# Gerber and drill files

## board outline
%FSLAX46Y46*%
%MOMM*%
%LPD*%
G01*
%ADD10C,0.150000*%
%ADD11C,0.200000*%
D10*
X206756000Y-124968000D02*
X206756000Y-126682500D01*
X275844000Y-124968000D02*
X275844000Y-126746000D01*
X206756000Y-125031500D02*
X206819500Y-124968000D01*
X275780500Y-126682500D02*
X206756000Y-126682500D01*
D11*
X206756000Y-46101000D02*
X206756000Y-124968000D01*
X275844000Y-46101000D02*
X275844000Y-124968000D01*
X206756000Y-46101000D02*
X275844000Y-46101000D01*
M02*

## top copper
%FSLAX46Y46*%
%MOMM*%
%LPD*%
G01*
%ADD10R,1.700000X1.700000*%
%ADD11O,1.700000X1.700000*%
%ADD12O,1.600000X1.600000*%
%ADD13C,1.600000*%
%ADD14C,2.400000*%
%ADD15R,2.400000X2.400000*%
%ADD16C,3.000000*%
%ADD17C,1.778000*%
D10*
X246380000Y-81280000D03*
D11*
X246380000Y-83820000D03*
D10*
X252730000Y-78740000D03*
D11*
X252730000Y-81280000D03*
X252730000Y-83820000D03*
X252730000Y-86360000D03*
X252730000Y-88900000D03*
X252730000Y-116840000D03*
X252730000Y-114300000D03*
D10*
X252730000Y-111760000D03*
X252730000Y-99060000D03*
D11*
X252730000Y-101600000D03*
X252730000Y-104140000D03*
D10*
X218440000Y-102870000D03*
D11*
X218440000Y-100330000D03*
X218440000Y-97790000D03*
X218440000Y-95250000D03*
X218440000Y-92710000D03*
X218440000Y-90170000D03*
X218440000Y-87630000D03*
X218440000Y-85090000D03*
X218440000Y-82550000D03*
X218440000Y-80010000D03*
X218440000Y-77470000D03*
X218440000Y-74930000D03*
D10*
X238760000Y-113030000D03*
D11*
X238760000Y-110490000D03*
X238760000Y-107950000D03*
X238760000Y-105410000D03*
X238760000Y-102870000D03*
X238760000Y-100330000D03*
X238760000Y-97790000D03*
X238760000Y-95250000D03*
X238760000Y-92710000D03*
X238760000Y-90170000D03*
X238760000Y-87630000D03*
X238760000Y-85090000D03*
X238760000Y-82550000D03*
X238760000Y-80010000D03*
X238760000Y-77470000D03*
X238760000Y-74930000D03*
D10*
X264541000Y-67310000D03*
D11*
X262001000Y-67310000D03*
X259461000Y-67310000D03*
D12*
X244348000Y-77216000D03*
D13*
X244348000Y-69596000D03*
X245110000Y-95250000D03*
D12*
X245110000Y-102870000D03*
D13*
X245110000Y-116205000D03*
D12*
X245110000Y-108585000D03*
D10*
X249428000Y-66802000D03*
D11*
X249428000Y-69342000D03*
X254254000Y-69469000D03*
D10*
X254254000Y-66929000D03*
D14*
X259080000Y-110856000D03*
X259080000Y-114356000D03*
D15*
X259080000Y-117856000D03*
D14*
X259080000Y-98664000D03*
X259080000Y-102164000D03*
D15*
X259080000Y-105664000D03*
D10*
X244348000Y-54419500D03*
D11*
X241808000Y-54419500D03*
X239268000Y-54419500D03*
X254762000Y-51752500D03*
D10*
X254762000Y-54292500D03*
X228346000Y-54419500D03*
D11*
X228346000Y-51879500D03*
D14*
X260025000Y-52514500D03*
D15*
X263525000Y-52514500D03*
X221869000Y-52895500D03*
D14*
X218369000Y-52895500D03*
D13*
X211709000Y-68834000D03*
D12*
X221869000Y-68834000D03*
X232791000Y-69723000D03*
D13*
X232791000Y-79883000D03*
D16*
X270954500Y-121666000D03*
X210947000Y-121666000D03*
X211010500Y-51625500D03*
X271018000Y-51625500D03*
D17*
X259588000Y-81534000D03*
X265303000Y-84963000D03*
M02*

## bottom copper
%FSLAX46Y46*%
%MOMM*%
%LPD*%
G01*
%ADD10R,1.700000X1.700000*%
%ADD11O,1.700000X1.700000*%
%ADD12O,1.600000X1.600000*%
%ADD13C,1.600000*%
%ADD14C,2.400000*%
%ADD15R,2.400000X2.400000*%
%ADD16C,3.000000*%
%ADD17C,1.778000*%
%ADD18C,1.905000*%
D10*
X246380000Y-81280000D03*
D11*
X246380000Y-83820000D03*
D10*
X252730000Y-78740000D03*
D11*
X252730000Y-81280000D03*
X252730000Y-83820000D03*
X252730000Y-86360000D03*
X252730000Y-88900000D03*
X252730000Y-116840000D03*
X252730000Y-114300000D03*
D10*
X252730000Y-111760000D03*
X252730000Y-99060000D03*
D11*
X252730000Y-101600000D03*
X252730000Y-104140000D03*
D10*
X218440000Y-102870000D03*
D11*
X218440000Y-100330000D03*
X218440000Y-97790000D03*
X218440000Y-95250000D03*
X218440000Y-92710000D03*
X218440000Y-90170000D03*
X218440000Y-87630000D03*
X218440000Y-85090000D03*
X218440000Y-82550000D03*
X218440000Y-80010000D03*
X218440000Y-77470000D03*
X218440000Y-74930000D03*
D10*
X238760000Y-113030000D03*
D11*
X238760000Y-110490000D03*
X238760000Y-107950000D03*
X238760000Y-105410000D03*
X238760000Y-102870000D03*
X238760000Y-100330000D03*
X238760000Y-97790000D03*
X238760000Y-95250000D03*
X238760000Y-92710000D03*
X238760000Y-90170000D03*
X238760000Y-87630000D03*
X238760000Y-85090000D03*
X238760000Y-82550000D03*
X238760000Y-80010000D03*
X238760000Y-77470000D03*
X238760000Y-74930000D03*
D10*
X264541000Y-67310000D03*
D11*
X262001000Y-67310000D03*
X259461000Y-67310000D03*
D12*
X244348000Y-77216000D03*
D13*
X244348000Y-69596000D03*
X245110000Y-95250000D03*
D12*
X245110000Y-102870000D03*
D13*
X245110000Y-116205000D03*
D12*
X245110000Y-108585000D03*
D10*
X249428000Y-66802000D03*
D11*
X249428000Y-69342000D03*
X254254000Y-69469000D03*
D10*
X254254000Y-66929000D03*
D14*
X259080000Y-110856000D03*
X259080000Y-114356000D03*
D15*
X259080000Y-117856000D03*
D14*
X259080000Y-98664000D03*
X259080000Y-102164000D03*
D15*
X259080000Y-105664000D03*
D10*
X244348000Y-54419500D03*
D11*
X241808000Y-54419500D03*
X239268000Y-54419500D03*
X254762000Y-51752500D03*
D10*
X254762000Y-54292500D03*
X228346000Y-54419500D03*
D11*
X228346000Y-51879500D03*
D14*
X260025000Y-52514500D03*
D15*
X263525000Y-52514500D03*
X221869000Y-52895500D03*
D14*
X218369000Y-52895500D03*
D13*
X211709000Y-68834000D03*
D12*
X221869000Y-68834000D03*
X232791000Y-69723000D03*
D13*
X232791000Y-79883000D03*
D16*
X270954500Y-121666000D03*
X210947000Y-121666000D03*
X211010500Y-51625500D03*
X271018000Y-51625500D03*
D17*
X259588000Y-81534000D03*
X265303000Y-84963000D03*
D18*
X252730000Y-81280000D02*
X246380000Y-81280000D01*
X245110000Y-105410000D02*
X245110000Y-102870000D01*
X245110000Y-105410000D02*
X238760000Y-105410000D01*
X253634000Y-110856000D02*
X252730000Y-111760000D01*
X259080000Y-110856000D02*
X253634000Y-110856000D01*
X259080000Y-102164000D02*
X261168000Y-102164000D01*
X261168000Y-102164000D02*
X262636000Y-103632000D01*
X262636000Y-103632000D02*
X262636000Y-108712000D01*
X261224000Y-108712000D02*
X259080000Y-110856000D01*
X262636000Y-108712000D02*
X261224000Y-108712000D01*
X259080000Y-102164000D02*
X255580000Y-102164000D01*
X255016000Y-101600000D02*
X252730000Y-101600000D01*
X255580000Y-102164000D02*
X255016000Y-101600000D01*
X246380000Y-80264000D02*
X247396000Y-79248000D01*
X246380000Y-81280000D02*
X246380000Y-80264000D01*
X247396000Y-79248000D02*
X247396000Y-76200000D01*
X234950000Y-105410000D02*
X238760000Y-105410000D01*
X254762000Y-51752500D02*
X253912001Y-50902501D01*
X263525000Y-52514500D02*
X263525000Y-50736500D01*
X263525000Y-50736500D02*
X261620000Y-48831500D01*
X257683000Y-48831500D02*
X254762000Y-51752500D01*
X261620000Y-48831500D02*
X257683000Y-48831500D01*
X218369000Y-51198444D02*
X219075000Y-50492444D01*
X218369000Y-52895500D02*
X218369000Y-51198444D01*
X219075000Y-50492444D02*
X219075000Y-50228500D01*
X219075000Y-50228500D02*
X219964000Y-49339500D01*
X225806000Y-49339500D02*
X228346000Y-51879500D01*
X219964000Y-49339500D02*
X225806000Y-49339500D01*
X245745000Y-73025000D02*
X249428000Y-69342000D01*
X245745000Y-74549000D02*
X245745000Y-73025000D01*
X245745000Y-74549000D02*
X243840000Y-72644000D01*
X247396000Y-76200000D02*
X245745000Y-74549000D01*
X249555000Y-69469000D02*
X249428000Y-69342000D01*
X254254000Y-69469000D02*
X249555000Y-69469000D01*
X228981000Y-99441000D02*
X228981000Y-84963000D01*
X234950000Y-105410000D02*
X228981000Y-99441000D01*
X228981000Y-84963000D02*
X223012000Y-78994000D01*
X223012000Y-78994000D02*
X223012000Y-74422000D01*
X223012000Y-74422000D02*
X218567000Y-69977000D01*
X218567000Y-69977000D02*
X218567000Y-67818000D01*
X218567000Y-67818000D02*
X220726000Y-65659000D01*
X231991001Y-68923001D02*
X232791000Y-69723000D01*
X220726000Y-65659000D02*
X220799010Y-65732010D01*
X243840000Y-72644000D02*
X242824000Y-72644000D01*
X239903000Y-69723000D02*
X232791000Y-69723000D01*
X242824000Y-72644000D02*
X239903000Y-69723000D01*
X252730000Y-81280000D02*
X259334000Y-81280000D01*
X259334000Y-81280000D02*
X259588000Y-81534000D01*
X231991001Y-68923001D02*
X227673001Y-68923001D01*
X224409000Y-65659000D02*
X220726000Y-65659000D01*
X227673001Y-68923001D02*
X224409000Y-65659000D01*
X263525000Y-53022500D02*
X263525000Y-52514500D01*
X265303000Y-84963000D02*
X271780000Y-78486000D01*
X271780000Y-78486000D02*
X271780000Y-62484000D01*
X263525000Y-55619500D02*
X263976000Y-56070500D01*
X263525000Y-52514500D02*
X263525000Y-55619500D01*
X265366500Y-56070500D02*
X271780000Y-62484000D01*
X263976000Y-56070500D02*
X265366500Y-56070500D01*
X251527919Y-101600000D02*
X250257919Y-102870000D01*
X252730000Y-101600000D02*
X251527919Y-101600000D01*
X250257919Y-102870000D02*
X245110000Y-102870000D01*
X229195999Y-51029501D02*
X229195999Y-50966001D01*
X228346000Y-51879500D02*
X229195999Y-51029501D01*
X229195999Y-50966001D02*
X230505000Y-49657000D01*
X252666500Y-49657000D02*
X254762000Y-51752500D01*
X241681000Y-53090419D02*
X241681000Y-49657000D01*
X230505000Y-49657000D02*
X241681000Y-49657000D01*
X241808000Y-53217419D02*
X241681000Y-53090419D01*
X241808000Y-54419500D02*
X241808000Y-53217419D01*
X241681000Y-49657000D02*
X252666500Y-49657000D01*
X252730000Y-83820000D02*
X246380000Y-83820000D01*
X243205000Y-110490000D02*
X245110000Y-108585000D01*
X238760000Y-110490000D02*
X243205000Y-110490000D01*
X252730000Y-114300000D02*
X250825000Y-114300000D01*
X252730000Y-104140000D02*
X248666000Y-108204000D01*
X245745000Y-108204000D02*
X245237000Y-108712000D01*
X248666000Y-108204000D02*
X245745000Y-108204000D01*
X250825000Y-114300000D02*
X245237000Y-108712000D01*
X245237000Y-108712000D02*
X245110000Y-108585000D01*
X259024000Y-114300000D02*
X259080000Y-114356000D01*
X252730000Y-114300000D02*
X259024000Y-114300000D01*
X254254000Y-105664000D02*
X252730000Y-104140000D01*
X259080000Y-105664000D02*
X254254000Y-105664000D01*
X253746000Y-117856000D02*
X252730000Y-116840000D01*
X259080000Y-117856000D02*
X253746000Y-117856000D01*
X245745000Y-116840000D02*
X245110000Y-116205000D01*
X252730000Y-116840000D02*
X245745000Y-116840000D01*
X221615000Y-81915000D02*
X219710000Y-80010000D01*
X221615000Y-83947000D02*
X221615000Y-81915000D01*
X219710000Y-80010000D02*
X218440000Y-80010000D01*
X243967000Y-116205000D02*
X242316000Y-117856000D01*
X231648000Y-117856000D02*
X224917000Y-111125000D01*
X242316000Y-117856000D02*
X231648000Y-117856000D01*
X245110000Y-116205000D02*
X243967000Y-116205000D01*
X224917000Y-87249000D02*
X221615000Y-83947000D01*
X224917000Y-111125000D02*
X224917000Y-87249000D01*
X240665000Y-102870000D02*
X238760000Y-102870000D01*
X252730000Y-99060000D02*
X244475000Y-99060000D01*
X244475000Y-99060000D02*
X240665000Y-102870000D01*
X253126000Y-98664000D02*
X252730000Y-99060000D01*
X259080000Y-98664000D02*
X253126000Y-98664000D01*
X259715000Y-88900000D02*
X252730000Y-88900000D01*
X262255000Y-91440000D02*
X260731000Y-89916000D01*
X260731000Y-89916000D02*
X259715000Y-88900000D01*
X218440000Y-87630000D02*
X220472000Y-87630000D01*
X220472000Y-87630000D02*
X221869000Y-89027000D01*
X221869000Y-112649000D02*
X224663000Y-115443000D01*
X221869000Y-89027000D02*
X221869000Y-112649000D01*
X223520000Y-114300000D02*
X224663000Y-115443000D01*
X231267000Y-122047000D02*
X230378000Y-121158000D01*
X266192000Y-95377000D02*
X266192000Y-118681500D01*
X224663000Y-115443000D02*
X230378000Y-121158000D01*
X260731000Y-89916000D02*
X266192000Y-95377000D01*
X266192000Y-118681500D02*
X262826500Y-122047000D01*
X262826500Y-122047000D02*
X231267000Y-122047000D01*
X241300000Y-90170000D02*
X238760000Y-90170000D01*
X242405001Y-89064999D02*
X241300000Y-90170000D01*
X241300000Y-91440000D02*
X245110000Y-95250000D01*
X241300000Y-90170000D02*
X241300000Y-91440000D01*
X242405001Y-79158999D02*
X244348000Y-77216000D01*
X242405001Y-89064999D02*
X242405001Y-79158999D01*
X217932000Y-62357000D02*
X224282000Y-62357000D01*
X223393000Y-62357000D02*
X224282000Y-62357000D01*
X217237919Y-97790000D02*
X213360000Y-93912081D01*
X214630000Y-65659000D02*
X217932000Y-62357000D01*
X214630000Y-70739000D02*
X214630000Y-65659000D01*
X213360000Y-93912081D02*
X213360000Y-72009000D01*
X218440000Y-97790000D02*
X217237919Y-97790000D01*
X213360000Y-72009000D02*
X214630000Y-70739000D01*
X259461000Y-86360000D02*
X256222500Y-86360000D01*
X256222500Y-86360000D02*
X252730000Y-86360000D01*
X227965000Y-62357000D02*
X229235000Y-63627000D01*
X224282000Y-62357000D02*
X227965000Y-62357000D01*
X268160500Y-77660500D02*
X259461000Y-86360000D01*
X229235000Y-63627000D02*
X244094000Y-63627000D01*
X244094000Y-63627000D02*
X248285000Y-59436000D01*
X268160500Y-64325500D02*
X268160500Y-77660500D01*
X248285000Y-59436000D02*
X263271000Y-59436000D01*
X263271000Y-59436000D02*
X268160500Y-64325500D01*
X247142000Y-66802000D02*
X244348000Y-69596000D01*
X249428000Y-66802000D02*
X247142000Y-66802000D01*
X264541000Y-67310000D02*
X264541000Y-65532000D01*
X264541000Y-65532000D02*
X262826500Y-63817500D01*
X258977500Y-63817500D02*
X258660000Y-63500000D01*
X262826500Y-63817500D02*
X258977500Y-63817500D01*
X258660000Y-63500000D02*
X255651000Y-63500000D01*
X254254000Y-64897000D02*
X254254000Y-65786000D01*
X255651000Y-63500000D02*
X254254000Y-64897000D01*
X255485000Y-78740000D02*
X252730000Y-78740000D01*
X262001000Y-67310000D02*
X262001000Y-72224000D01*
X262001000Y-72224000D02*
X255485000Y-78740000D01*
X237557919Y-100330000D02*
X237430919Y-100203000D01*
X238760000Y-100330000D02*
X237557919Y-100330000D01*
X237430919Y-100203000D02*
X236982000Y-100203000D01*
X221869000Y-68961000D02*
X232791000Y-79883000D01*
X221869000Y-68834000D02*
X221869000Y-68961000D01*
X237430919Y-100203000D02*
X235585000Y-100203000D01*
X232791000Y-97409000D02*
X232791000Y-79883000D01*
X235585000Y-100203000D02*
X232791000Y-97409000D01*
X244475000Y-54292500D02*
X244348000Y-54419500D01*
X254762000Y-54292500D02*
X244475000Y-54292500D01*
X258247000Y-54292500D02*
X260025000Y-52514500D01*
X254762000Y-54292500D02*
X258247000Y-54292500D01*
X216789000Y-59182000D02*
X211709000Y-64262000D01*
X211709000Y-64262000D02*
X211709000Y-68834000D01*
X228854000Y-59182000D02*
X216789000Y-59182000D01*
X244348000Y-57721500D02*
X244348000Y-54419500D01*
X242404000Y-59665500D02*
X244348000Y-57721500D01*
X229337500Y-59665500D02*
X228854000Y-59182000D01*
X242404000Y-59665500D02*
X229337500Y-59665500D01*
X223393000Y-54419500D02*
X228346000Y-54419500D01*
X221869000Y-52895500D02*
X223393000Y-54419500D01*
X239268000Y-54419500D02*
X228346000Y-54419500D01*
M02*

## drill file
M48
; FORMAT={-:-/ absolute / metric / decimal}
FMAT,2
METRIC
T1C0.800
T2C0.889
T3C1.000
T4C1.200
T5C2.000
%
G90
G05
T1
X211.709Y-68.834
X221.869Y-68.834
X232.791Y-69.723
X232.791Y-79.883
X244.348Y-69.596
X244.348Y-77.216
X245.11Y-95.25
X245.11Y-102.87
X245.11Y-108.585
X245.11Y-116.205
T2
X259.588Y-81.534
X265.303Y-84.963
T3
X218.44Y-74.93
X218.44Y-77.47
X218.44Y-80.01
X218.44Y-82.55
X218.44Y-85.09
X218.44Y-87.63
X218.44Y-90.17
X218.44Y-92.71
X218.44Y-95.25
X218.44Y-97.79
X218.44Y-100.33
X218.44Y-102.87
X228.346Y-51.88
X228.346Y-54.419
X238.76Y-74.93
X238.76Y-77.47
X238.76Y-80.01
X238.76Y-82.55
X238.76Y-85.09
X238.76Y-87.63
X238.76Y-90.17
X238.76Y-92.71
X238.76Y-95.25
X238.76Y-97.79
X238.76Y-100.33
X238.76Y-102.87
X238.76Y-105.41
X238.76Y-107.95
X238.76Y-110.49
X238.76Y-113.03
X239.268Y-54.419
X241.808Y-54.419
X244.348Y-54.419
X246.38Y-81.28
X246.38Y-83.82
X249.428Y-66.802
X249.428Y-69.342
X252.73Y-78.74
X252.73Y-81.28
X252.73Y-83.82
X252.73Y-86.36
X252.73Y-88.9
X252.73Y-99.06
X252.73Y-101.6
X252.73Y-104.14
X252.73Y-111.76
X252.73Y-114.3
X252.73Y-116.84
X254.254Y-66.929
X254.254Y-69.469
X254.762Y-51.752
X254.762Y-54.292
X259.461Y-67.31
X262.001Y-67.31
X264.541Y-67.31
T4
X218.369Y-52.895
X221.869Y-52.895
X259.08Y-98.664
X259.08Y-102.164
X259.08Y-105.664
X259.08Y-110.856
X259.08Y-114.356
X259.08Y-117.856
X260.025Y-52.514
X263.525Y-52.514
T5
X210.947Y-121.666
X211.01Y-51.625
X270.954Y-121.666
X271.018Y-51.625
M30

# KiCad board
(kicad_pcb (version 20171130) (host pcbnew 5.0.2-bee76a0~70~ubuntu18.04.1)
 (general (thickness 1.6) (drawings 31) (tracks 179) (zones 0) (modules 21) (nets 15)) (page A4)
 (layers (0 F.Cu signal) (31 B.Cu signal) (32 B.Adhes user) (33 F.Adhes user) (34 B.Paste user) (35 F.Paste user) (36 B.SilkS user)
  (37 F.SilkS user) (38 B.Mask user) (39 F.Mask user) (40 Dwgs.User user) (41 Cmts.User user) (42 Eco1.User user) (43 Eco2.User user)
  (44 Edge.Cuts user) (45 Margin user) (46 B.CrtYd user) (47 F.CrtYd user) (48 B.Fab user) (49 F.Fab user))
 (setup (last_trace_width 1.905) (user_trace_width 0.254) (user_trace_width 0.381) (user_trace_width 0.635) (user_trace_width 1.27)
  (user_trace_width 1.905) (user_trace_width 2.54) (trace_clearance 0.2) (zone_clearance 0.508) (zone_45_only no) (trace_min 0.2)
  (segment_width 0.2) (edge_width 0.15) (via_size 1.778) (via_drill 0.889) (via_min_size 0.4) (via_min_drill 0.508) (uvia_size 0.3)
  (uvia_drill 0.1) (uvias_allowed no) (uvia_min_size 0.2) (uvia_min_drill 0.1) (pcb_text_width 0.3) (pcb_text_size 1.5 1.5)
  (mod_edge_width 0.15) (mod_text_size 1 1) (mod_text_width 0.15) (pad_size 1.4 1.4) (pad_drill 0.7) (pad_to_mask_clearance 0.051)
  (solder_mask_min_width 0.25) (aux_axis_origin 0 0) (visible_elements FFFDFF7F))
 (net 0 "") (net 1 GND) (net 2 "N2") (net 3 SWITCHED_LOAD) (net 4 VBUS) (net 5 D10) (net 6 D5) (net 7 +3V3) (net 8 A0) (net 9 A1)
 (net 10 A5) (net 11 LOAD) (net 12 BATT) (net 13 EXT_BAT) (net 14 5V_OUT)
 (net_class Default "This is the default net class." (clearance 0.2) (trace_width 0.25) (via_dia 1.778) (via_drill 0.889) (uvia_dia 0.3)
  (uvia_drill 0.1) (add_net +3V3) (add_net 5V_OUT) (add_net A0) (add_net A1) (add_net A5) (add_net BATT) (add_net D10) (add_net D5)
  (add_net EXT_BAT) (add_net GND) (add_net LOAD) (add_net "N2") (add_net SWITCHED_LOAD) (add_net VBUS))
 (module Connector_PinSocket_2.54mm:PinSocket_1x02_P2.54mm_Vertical (layer F.Cu) (at 246.38 81.28)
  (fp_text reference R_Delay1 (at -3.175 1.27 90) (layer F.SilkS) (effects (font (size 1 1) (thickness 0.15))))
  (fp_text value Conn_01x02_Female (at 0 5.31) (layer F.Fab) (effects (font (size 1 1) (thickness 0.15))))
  (pad 1 thru_hole rect (at 0 0) (size 1.7 1.7) (drill 1) (layers *.Cu *.Mask) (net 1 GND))
  (pad 2 thru_hole oval (at 0 2.54) (size 1.7 1.7) (drill 1) (layers *.Cu *.Mask) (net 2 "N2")))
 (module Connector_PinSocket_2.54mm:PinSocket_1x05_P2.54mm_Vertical (layer F.Cu) (at 252.73 78.74)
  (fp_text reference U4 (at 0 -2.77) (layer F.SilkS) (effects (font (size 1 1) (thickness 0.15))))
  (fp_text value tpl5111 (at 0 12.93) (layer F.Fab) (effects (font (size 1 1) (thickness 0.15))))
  (pad 1 thru_hole rect (at 0 0) (size 1.7 1.7) (drill 1) (layers *.Cu *.Mask) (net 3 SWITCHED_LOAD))
  (pad 2 thru_hole oval (at 0 2.54) (size 1.7 1.7) (drill 1) (layers *.Cu *.Mask) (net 1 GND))
  (pad 3 thru_hole oval (at 0 5.08) (size 1.7 1.7) (drill 1) (layers *.Cu *.Mask) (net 2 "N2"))
  (pad 4 thru_hole oval (at 0 7.62) (size 1.7 1.7) (drill 1) (layers *.Cu *.Mask) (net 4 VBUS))
  (pad 5 thru_hole oval (at 0 10.16) (size 1.7 1.7) (drill 1) (layers *.Cu *.Mask) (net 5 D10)))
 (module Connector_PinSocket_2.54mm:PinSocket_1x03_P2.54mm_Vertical (layer F.Cu) (at 252.73 111.76)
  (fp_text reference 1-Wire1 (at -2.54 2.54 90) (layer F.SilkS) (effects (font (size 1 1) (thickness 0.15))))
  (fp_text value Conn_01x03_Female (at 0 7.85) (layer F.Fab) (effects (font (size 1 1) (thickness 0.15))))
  (pad 3 thru_hole oval (at 0 5.08) (size 1.7 1.7) (drill 1) (layers *.Cu *.Mask) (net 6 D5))
  (pad 2 thru_hole oval (at 0 2.54) (size 1.7 1.7) (drill 1) (layers *.Cu *.Mask) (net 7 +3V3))
  (pad 1 thru_hole rect (at 0 0) (size 1.7 1.7) (drill 1) (layers *.Cu *.Mask) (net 1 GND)))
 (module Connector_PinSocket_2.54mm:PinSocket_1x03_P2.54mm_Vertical (layer F.Cu) (at 252.73 99.06)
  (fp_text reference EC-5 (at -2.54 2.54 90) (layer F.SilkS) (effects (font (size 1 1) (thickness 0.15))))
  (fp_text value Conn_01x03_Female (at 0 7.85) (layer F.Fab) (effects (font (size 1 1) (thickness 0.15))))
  (pad 1 thru_hole rect (at 0 0) (size 1.7 1.7) (drill 1) (layers *.Cu *.Mask) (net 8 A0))
  (pad 2 thru_hole oval (at 0 2.54) (size 1.7 1.7) (drill 1) (layers *.Cu *.Mask) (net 1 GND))
  (pad 3 thru_hole oval (at 0 5.08) (size 1.7 1.7) (drill 1) (layers *.Cu *.Mask) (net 7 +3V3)))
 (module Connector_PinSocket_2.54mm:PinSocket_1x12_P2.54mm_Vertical (layer F.Cu) (at 218.44 102.87 180)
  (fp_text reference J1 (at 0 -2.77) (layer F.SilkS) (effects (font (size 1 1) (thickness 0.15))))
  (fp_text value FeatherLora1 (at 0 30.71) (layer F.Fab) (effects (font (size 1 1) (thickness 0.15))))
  (pad 1 thru_hole rect (at 0 0 180) (size 1.7 1.7) (drill 1) (layers *.Cu *.Mask))
  (pad 2 thru_hole oval (at 0 2.54 180) (size 1.7 1.7) (drill 1) (layers *.Cu *.Mask))
  (pad 3 thru_hole oval (at 0 5.08 180) (size 1.7 1.7) (drill 1) (layers *.Cu *.Mask) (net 4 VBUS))
  (pad 4 thru_hole oval (at 0 7.62 180) (size 1.7 1.7) (drill 1) (layers *.Cu *.Mask))
  (pad 5 thru_hole oval (at 0 10.16 180) (size 1.7 1.7) (drill 1) (layers *.Cu *.Mask))
  (pad 6 thru_hole oval (at 0 12.7 180) (size 1.7 1.7) (drill 1) (layers *.Cu *.Mask))
  (pad 7 thru_hole oval (at 0 15.24 180) (size 1.7 1.7) (drill 1) (layers *.Cu *.Mask) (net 5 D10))
  (pad 8 thru_hole oval (at 0 17.78 180) (size 1.7 1.7) (drill 1) (layers *.Cu *.Mask))
  (pad 9 thru_hole oval (at 0 20.32 180) (size 1.7 1.7) (drill 1) (layers *.Cu *.Mask))
  (pad 10 thru_hole oval (at 0 22.86 180) (size 1.7 1.7) (drill 1) (layers *.Cu *.Mask) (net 6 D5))
  (pad 11 thru_hole oval (at 0 25.4 180) (size 1.7 1.7) (drill 1) (layers *.Cu *.Mask))
  (pad 12 thru_hole oval (at 0 27.94 180) (size 1.7 1.7) (drill 1) (layers *.Cu *.Mask)))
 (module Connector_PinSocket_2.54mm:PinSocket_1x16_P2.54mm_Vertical (layer F.Cu) (at 238.76 113.03 180)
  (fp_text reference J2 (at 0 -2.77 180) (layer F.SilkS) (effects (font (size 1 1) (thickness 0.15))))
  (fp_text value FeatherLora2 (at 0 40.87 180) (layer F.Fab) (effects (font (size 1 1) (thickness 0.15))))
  (pad 1 thru_hole rect (at 0 0 180) (size 1.7 1.7) (drill 1) (layers *.Cu *.Mask))
  (pad 2 thru_hole oval (at 0 2.54 180) (size 1.7 1.7) (drill 1) (layers *.Cu *.Mask) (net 7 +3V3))
  (pad 3 thru_hole oval (at 0 5.08 180) (size 1.7 1.7) (drill 1) (layers *.Cu *.Mask))
  (pad 4 thru_hole oval (at 0 7.62 180) (size 1.7 1.7) (drill 1) (layers *.Cu *.Mask) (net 1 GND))
  (pad 5 thru_hole oval (at 0 10.16 180) (size 1.7 1.7) (drill 1) (layers *.Cu *.Mask) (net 8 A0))
  (pad 6 thru_hole oval (at 0 12.7 180) (size 1.7 1.7) (drill 1) (layers *.Cu *.Mask) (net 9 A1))
  (pad 7 thru_hole oval (at 0 15.24 180) (size 1.7 1.7) (drill 1) (layers *.Cu *.Mask))
  (pad 8 thru_hole oval (at 0 17.78 180) (size 1.7 1.7) (drill 1) (layers *.Cu *.Mask))
  (pad 9 thru_hole oval (at 0 20.32 180) (size 1.7 1.7) (drill 1) (layers *.Cu *.Mask))
  (pad 10 thru_hole oval (at 0 22.86 180) (size 1.7 1.7) (drill 1) (layers *.Cu *.Mask) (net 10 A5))
  (pad 11 thru_hole oval (at 0 25.4 180) (size 1.7 1.7) (drill 1) (layers *.Cu *.Mask))
  (pad 12 thru_hole oval (at 0 27.94 180) (size 1.7 1.7) (drill 1) (layers *.Cu *.Mask))
  (pad 13 thru_hole oval (at 0 30.48 180) (size 1.7 1.7) (drill 1) (layers *.Cu *.Mask))
  (pad 14 thru_hole oval (at 0 33.02 180) (size 1.7 1.7) (drill 1) (layers *.Cu *.Mask))
  (pad 15 thru_hole oval (at 0 35.56 180) (size 1.7 1.7) (drill 1) (layers *.Cu *.Mask))
  (pad 16 thru_hole oval (at 0 38.1 180) (size 1.7 1.7) (drill 1) (layers *.Cu *.Mask)))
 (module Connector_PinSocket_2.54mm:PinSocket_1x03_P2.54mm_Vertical (layer F.Cu) (at 264.541 67.31 270)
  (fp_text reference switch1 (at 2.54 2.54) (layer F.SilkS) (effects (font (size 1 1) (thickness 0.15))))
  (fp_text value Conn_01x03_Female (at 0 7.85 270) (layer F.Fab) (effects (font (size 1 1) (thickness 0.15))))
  (pad 1 thru_hole rect (at 0 0 270) (size 1.7 1.7) (drill 1) (layers *.Cu *.Mask) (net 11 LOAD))
  (pad 2 thru_hole oval (at 0 2.54 270) (size 1.7 1.7) (drill 1) (layers *.Cu *.Mask) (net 3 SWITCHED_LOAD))
  (pad 3 thru_hole oval (at 0 5.08 270) (size 1.7 1.7) (drill 1) (layers *.Cu *.Mask)))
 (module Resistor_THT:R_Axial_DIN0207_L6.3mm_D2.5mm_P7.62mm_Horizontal (layer F.Cu) (at 244.348 69.596 270)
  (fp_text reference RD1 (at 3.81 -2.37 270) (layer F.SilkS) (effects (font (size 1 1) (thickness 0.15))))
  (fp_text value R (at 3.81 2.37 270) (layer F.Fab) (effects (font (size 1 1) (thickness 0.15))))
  (pad 2 thru_hole oval (at 7.62 0 270) (size 1.6 1.6) (drill 0.8) (layers *.Cu *.Mask) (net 10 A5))
  (pad 1 thru_hole circle (at 0 0 270) (size 1.6 1.6) (drill 0.8) (layers *.Cu *.Mask) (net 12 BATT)))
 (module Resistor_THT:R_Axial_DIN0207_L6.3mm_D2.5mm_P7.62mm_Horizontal (layer F.Cu) (at 245.11 95.25 270)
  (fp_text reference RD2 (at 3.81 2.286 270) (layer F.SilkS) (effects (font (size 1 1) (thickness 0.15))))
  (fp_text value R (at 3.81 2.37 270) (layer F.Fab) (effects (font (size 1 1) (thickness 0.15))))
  (pad 1 thru_hole circle (at 0 0 270) (size 1.6 1.6) (drill 0.8) (layers *.Cu *.Mask) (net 10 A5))
  (pad 2 thru_hole oval (at 7.62 0 270) (size 1.6 1.6) (drill 0.8) (layers *.Cu *.Mask) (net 1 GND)))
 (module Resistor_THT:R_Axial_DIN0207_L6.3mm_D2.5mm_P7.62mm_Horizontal (layer F.Cu) (at 245.11 116.205 90)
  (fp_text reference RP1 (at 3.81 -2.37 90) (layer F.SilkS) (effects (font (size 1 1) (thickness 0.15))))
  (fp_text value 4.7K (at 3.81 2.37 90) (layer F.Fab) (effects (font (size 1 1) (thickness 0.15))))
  (pad 1 thru_hole circle (at 0 0 90) (size 1.6 1.6) (drill 0.8) (layers *.Cu *.Mask) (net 6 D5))
  (pad 2 thru_hole oval (at 7.62 0 90) (size 1.6 1.6) (drill 0.8) (layers *.Cu *.Mask) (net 7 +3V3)))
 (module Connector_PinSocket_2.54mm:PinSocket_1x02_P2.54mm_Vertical (layer F.Cu) (at 249.428 66.802)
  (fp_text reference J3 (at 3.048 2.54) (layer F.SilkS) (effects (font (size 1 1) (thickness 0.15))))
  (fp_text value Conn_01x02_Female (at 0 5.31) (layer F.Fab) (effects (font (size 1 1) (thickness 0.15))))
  (pad 1 thru_hole rect (at 0 0) (size 1.7 1.7) (drill 1) (layers *.Cu *.Mask) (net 12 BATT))
  (pad 2 thru_hole oval (at 0 2.54) (size 1.7 1.7) (drill 1) (layers *.Cu *.Mask) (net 1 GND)))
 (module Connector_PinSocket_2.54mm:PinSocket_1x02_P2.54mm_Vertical (layer F.Cu) (at 254.254 66.929)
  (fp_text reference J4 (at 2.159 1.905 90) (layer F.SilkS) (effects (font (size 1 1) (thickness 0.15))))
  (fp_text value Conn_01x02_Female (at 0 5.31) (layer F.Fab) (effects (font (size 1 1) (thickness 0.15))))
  (pad 2 thru_hole oval (at 0 2.54) (size 1.7 1.7) (drill 1) (layers *.Cu *.Mask) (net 1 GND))
  (pad 1 thru_hole rect (at 0 0) (size 1.7 1.7) (drill 1) (layers *.Cu *.Mask) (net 11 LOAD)))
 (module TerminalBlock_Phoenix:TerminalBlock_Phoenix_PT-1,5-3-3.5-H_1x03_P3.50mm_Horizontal (layer F.Cu) (at 259.08 117.856 90)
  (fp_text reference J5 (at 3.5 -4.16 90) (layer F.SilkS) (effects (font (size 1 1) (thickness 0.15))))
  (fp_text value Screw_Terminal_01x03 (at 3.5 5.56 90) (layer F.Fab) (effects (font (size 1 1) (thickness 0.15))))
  (pad 3 thru_hole circle (at 7 0 90) (size 2.4 2.4) (drill 1.2) (layers *.Cu *.Mask) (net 1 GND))
  (pad 2 thru_hole circle (at 3.5 0 90) (size 2.4 2.4) (drill 1.2) (layers *.Cu *.Mask) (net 7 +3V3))
  (pad 1 thru_hole rect (at 0 0 90) (size 2.4 2.4) (drill 1.2) (layers *.Cu *.Mask) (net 6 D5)))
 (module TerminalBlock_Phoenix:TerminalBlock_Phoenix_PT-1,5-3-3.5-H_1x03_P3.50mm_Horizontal (layer F.Cu) (at 259.08 105.664 90)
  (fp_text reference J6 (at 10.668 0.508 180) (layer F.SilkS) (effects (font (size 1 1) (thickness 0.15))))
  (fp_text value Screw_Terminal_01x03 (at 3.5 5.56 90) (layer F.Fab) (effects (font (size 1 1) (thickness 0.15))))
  (pad 3 thru_hole circle (at 7 0 90) (size 2.4 2.4) (drill 1.2) (layers *.Cu *.Mask) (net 8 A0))
  (pad 2 thru_hole circle (at 3.5 0 90) (size 2.4 2.4) (drill 1.2) (layers *.Cu *.Mask) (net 1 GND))
  (pad 1 thru_hole rect (at 0 0 90) (size 2.4 2.4) (drill 1.2) (layers *.Cu *.Mask) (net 7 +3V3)))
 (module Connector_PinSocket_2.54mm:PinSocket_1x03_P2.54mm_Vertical (layer F.Cu) (at 244.348 54.4195 270)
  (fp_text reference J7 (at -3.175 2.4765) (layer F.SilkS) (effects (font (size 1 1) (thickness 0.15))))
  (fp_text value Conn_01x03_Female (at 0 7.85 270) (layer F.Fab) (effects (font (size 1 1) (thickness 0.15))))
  (pad 1 thru_hole rect (at 0 0 270) (size 1.7 1.7) (drill 1) (layers *.Cu *.Mask) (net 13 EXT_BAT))
  (pad 2 thru_hole oval (at 0 2.54 270) (size 1.7 1.7) (drill 1) (layers *.Cu *.Mask) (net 1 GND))
  (pad 3 thru_hole oval (at 0 5.08 270) (size 1.7 1.7) (drill 1) (layers *.Cu *.Mask) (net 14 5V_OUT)))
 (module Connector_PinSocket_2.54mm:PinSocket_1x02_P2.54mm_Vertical (layer F.Cu) (at 254.762 54.2925 180)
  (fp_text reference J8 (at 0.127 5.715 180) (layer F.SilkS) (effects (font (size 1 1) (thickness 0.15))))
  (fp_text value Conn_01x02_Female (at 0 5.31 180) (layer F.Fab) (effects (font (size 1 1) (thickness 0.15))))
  (pad 2 thru_hole oval (at 0 2.54 180) (size 1.7 1.7) (drill 1) (layers *.Cu *.Mask) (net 1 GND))
  (pad 1 thru_hole rect (at 0 0 180) (size 1.7 1.7) (drill 1) (layers *.Cu *.Mask) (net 13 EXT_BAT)))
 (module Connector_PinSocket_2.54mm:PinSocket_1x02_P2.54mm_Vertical (layer F.Cu) (at 228.346 54.4195 180)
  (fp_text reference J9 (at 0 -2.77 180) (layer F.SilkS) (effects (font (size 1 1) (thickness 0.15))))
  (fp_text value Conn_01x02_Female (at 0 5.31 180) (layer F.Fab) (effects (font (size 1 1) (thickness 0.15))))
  (pad 1 thru_hole rect (at 0 0 180) (size 1.7 1.7) (drill 1) (layers *.Cu *.Mask) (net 14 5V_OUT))
  (pad 2 thru_hole oval (at 0 2.54 180) (size 1.7 1.7) (drill 1) (layers *.Cu *.Mask) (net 1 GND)))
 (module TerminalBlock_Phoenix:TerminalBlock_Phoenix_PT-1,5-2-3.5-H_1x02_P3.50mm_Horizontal (layer F.Cu) (at 263.525 52.5145 180)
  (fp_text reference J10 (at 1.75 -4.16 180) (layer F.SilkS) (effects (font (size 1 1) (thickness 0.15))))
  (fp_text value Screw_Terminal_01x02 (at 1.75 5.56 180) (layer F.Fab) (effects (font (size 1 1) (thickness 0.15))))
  (pad 2 thru_hole circle (at 3.5 0 180) (size 2.4 2.4) (drill 1.2) (layers *.Cu *.Mask) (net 13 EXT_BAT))
  (pad 1 thru_hole rect (at 0 0 180) (size 2.4 2.4) (drill 1.2) (layers *.Cu *.Mask) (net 1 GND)))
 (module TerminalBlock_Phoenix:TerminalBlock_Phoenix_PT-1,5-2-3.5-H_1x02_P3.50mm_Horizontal (layer F.Cu) (at 221.869 52.8955 180)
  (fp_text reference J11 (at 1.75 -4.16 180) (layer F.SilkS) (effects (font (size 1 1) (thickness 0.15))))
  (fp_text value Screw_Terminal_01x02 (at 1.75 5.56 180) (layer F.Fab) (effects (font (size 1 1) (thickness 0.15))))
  (pad 1 thru_hole rect (at 0 0 180) (size 2.4 2.4) (drill 1.2) (layers *.Cu *.Mask) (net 14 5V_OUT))
  (pad 2 thru_hole circle (at 3.5 0 180) (size 2.4 2.4) (drill 1.2) (layers *.Cu *.Mask) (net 1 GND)))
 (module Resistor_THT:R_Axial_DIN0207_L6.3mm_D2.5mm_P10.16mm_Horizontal (layer F.Cu) (at 211.709 68.834)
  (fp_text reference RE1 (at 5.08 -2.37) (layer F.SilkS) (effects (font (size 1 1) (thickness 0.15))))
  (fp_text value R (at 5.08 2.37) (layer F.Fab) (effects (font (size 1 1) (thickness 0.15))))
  (pad 1 thru_hole circle (at 0 0) (size 1.6 1.6) (drill 0.8) (layers *.Cu *.Mask) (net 13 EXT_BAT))
  (pad 2 thru_hole oval (at 10.16 0) (size 1.6 1.6) (drill 0.8) (layers *.Cu *.Mask) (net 9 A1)))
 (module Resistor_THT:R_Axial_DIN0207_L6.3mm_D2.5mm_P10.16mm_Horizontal (layer F.Cu) (at 232.791 79.883 90)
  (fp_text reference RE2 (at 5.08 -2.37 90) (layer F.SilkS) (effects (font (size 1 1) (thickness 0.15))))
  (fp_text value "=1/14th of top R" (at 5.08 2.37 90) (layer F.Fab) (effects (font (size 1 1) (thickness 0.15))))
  (pad 2 thru_hole oval (at 10.16 0 90) (size 1.6 1.6) (drill 0.8) (layers *.Cu *.Mask) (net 1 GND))
  (pad 1 thru_hole circle (at 0 0 90) (size 1.6 1.6) (drill 0.8) (layers *.Cu *.Mask) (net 9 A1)))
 (gr_line (start 206.756 124.968) (end 206.756 126.6825) (layer Edge.Cuts) (width 0.15))
 (gr_line (start 275.844 124.968) (end 275.844 126.746) (layer Edge.Cuts) (width 0.15))
 (gr_line (start 206.756 125.0315) (end 206.8195 124.968) (layer Edge.Cuts) (width 0.15))
 (gr_line (start 275.7805 126.6825) (end 206.756 126.6825) (layer Edge.Cuts) (width 0.15))
 (gr_line (start 206.756 46.101) (end 206.756 124.968) (layer Edge.Cuts) (width 0.2))
 (gr_line (start 275.844 46.101) (end 275.844 124.968) (layer Edge.Cuts) (width 0.2))
 (gr_line (start 206.756 46.101) (end 275.844 46.101) (layer Edge.Cuts) (width 0.2))
 (via (at 270.9545 121.666) (size 3) (drill 2) (layers F.Cu B.Cu) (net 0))
 (via (at 210.947 121.666) (size 3) (drill 2) (layers F.Cu B.Cu) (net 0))
 (via (at 211.0105 51.6255) (size 3) (drill 2) (layers F.Cu B.Cu) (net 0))
 (via (at 271.018 51.6255) (size 3) (drill 2) (layers F.Cu B.Cu) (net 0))
 (segment (start 252.73 81.28) (end 246.38 81.28) (width 1.905) (layer B.Cu) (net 1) (status 30))
 (segment (start 245.11 105.41) (end 245.11 102.87) (width 1.905) (layer B.Cu) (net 1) (status 20))
 (segment (start 245.11 105.41) (end 238.76 105.41) (width 1.905) (layer B.Cu) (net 1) (status 20))
 (segment (start 253.634 110.856) (end 252.73 111.76) (width 1.905) (layer B.Cu) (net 1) (status 20))
 (segment (start 259.08 110.856) (end 253.634 110.856) (width 1.905) (layer B.Cu) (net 1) (status 10))
 (segment (start 259.08 102.164) (end 261.168 102.164) (width 1.905) (layer B.Cu) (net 1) (status 10))
 (segment (start 261.168 102.164) (end 262.636 103.632) (width 1.905) (layer B.Cu) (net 1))
 (segment (start 262.636 103.632) (end 262.636 108.712) (width 1.905) (layer B.Cu) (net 1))
 (segment (start 261.224 108.712) (end 259.08 110.856) (width 1.905) (layer B.Cu) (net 1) (status 20))
 (segment (start 262.636 108.712) (end 261.224 108.712) (width 1.905) (layer B.Cu) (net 1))
 (segment (start 259.08 102.164) (end 255.58 102.164) (width 1.905) (layer B.Cu) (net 1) (status 10))
 (segment (start 255.016 101.6) (end 252.73 101.6) (width 1.905) (layer B.Cu) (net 1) (status 20))
 (segment (start 255.58 102.164) (end 255.016 101.6) (width 1.905) (layer B.Cu) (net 1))
 (segment (start 246.38 80.264) (end 247.396 79.248) (width 1.905) (layer B.Cu) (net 1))
 (segment (start 246.38 81.28) (end 246.38 80.264) (width 1.905) (layer B.Cu) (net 1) (status 10))
 (segment (start 247.396 79.248) (end 247.396 76.2) (width 1.905) (layer B.Cu) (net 1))
 (segment (start 234.95 105.41) (end 238.76 105.41) (width 1.905) (layer B.Cu) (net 1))
 (segment (start 254.762 51.7525) (end 253.912001 50.902501) (width 1.905) (layer B.Cu) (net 1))
 (segment (start 263.525 52.5145) (end 263.525 50.7365) (width 1.905) (layer B.Cu) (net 1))
 (segment (start 263.525 50.7365) (end 261.62 48.8315) (width 1.905) (layer B.Cu) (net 1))
 (segment (start 257.683 48.8315) (end 254.762 51.7525) (width 1.905) (layer B.Cu) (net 1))
 (segment (start 261.62 48.8315) (end 257.683 48.8315) (width 1.905) (layer B.Cu) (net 1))
 (segment (start 218.369 51.198444) (end 219.075 50.492444) (width 1.905) (layer B.Cu) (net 1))
 (segment (start 218.369 52.8955) (end 218.369 51.198444) (width 1.905) (layer B.Cu) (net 1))
 (segment (start 219.075 50.492444) (end 219.075 50.2285) (width 1.905) (layer B.Cu) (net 1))
 (segment (start 219.075 50.2285) (end 219.964 49.3395) (width 1.905) (layer B.Cu) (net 1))
 (segment (start 225.806 49.3395) (end 228.346 51.8795) (width 1.905) (layer B.Cu) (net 1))
 (segment (start 219.964 49.3395) (end 225.806 49.3395) (width 1.905) (layer B.Cu) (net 1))
 (segment (start 245.745 73.025) (end 249.428 69.342) (width 1.905) (layer B.Cu) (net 1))
 (segment (start 245.745 74.549) (end 245.745 73.025) (width 1.905) (layer B.Cu) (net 1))
 (segment (start 245.745 74.549) (end 243.84 72.644) (width 1.905) (layer B.Cu) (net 1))
 (segment (start 247.396 76.2) (end 245.745 74.549) (width 1.905) (layer B.Cu) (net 1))
 (segment (start 249.555 69.469) (end 249.428 69.342) (width 1.905) (layer B.Cu) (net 1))
 (segment (start 254.254 69.469) (end 249.555 69.469) (width 1.905) (layer B.Cu) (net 1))
 (segment (start 228.981 99.441) (end 228.981 84.963) (width 1.905) (layer B.Cu) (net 1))
 (segment (start 234.95 105.41) (end 228.981 99.441) (width 1.905) (layer B.Cu) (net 1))
 (segment (start 228.981 84.963) (end 223.012 78.994) (width 1.905) (layer B.Cu) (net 1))
 (segment (start 223.012 78.994) (end 223.012 74.422) (width 1.905) (layer B.Cu) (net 1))
 (segment (start 223.012 74.422) (end 218.567 69.977) (width 1.905) (layer B.Cu) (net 1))
 (segment (start 218.567 69.977) (end 218.567 67.818) (width 1.905) (layer B.Cu) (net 1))
 (segment (start 218.567 67.818) (end 220.726 65.659) (width 1.905) (layer B.Cu) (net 1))
 (segment (start 231.991001 68.923001) (end 232.791 69.723) (width 1.905) (layer B.Cu) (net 1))
 (segment (start 220.726 65.659) (end 220.79901 65.73201) (width 1.905) (layer B.Cu) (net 1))
 (segment (start 243.84 72.644) (end 242.824 72.644) (width 1.905) (layer B.Cu) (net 1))
 (segment (start 239.903 69.723) (end 232.791 69.723) (width 1.905) (layer B.Cu) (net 1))
 (segment (start 242.824 72.644) (end 239.903 69.723) (width 1.905) (layer B.Cu) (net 1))
 (via (at 259.588 81.534) (size 1.778) (drill 0.889) (layers F.Cu B.Cu) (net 1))
 (segment (start 252.73 81.28) (end 259.334 81.28) (width 1.905) (layer B.Cu) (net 1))
 (segment (start 259.334 81.28) (end 259.588 81.534) (width 1.905) (layer B.Cu) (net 1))
 (via (at 265.303 84.963) (size 1.778) (drill 0.889) (layers F.Cu B.Cu) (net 1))
 (segment (start 231.991001 68.923001) (end 227.673001 68.923001) (width 1.905) (layer B.Cu) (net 1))
 (segment (start 224.409 65.659) (end 220.726 65.659) (width 1.905) (layer B.Cu) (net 1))
 (segment (start 227.673001 68.923001) (end 224.409 65.659) (width 1.905) (layer B.Cu) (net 1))
 (segment (start 263.525 53.0225) (end 263.525 52.5145) (width 1.905) (layer B.Cu) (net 1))
 (segment (start 265.303 84.963) (end 271.78 78.486) (width 1.905) (layer B.Cu) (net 1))
 (segment (start 271.78 78.486) (end 271.78 62.484) (width 1.905) (layer B.Cu) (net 1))
 (segment (start 263.525 55.6195) (end 263.976 56.0705) (width 1.905) (layer B.Cu) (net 1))
 (segment (start 263.525 52.5145) (end 263.525 55.6195) (width 1.905) (layer B.Cu) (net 1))
 (segment (start 265.3665 56.0705) (end 271.78 62.484) (width 1.905) (layer B.Cu) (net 1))
 (segment (start 263.976 56.0705) (end 265.3665 56.0705) (width 1.905) (layer B.Cu) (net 1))
 (segment (start 251.527919 101.6) (end 250.257919 102.87) (width 1.905) (layer B.Cu) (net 1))
 (segment (start 252.73 101.6) (end 251.527919 101.6) (width 1.905) (layer B.Cu) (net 1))
 (segment (start 250.257919 102.87) (end 245.11 102.87) (width 1.905) (layer B.Cu) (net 1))
 (segment (start 229.195999 51.029501) (end 229.195999 50.966001) (width 1.905) (layer B.Cu) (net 1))
 (segment (start 228.346 51.8795) (end 229.195999 51.029501) (width 1.905) (layer B.Cu) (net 1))
 (segment (start 229.195999 50.966001) (end 230.505 49.657) (width 1.905) (layer B.Cu) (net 1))
 (segment (start 252.6665 49.657) (end 254.762 51.7525) (width 1.905) (layer B.Cu) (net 1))
 (segment (start 241.681 53.090419) (end 241.681 49.657) (width 1.905) (layer B.Cu) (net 1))
 (segment (start 230.505 49.657) (end 241.681 49.657) (width 1.905) (layer B.Cu) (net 1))
 (segment (start 241.808 53.217419) (end 241.681 53.090419) (width 1.905) (layer B.Cu) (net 1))
 (segment (start 241.808 54.4195) (end 241.808 53.217419) (width 1.905) (layer B.Cu) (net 1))
 (segment (start 241.681 49.657) (end 252.6665 49.657) (width 1.905) (layer B.Cu) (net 1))
 (segment (start 252.73 83.82) (end 246.38 83.82) (width 1.905) (layer B.Cu) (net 2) (status 30))
 (segment (start 243.205 110.49) (end 245.11 108.585) (width 1.905) (layer B.Cu) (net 7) (status 20))
 (segment (start 238.76 110.49) (end 243.205 110.49) (width 1.905) (layer B.Cu) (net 7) (status 10))
 (segment (start 252.73 114.3) (end 250.825 114.3) (width 1.905) (layer B.Cu) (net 7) (status 10))
 (segment (start 252.73 104.14) (end 248.666 108.204) (width 1.905) (layer B.Cu) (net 7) (status 10))
 (segment (start 245.745 108.204) (end 245.237 108.712) (width 1.905) (layer B.Cu) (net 7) (status 30))
 (segment (start 248.666 108.204) (end 245.745 108.204) (width 1.905) (layer B.Cu) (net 7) (status 20))
 (segment (start 250.825 114.3) (end 245.237 108.712) (width 1.905) (layer B.Cu) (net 7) (status 20))
 (segment (start 245.237 108.712) (end 245.11 108.585) (width 1.905) (layer B.Cu) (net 7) (status 30))
 (segment (start 259.024 114.3) (end 259.08 114.356) (width 1.905) (layer B.Cu) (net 7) (status 30))
 (segment (start 252.73 114.3) (end 259.024 114.3) (width 1.905) (layer B.Cu) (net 7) (status 30))
 (segment (start 254.254 105.664) (end 252.73 104.14) (width 1.905) (layer B.Cu) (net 7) (status 20))
 (segment (start 259.08 105.664) (end 254.254 105.664) (width 1.905) (layer B.Cu) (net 7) (status 10))
 (segment (start 253.746 117.856) (end 252.73 116.84) (width 1.905) (layer B.Cu) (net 6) (status 20))
 (segment (start 259.08 117.856) (end 253.746 117.856) (width 1.905) (layer B.Cu) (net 6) (status 10))
 (segment (start 245.745 116.84) (end 245.11 116.205) (width 1.905) (layer B.Cu) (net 6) (status 20))
 (segment (start 252.73 116.84) (end 245.745 116.84) (width 1.905) (layer B.Cu) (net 6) (status 10))
 (segment (start 221.615 81.915) (end 219.71 80.01) (width 1.905) (layer B.Cu) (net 6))
 (segment (start 221.615 83.947) (end 221.615 81.915) (width 1.905) (layer B.Cu) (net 6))
 (segment (start 219.71 80.01) (end 218.44 80.01) (width 1.905) (layer B.Cu) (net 6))
 (segment (start 243.967 116.205) (end 242.316 117.856) (width 1.905) (layer B.Cu) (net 6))
 (segment (start 231.648 117.856) (end 224.917 111.125) (width 1.905) (layer B.Cu) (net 6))
 (segment (start 242.316 117.856) (end 231.648 117.856) (width 1.905) (layer B.Cu) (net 6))
 (segment (start 245.11 116.205) (end 243.967 116.205) (width 1.905) (layer B.Cu) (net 6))
 (segment (start 224.917 87.249) (end 221.615 83.947) (width 1.905) (layer B.Cu) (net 6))
 (segment (start 224.917 111.125) (end 224.917 87.249) (width 1.905) (layer B.Cu) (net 6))
 (segment (start 240.665 102.87) (end 238.76 102.87) (width 1.905) (layer B.Cu) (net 8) (status 20))
 (segment (start 252.73 99.06) (end 244.475 99.06) (width 1.905) (layer B.Cu) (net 8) (status 10))
 (segment (start 244.475 99.06) (end 240.665 102.87) (width 1.905) (layer B.Cu) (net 8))
 (segment (start 253.126 98.664) (end 252.73 99.06) (width 1.905) (layer B.Cu) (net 8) (status 30))
 (segment (start 259.08 98.664) (end 253.126 98.664) (width 1.905) (layer B.Cu) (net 8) (status 30))
 (segment (start 259.715 88.9) (end 252.73 88.9) (width 1.905) (layer B.Cu) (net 5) (status 20))
 (segment (start 262.255 91.44) (end 260.731 89.916) (width 1.905) (layer B.Cu) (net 5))
 (segment (start 260.731 89.916) (end 259.715 88.9) (width 1.905) (layer B.Cu) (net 5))
 (segment (start 218.44 87.63) (end 220.472 87.63) (width 1.905) (layer B.Cu) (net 5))
 (segment (start 220.472 87.63) (end 221.869 89.027) (width 1.905) (layer B.Cu) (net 5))
 (segment (start 221.869 112.649) (end 224.663 115.443) (width 1.905) (layer B.Cu) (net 5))
 (segment (start 221.869 89.027) (end 221.869 112.649) (width 1.905) (layer B.Cu) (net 5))
 (segment (start 223.52 114.3) (end 224.663 115.443) (width 1.905) (layer B.Cu) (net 5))
 (segment (start 231.267 122.047) (end 230.378 121.158) (width 1.905) (layer B.Cu) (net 5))
 (segment (start 266.192 95.377) (end 266.192 118.6815) (width 1.905) (layer B.Cu) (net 5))
 (segment (start 224.663 115.443) (end 230.378 121.158) (width 1.905) (layer B.Cu) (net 5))
 (segment (start 260.731 89.916) (end 266.192 95.377) (width 1.905) (layer B.Cu) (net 5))
 (segment (start 266.192 118.6815) (end 262.8265 122.047) (width 1.905) (layer B.Cu) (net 5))
 (segment (start 262.8265 122.047) (end 231.267 122.047) (width 1.905) (layer B.Cu) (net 5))
 (segment (start 241.3 90.17) (end 238.76 90.17) (width 1.905) (layer B.Cu) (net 10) (status 20))
 (segment (start 242.405001 89.064999) (end 241.3 90.17) (width 1.905) (layer B.Cu) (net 10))
 (segment (start 241.3 91.44) (end 245.11 95.25) (width 1.905) (layer B.Cu) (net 10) (status 20))
 (segment (start 241.3 90.17) (end 241.3 91.44) (width 1.905) (layer B.Cu) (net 10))
 (segment (start 242.405001 79.158999) (end 244.348 77.216) (width 1.905) (layer B.Cu) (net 10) (status 20))
 (segment (start 242.405001 89.064999) (end 242.405001 79.158999) (width 1.905) (layer B.Cu) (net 10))
 (segment (start 217.932 62.357) (end 224.282 62.357) (width 1.905) (layer B.Cu) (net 4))
 (segment (start 223.393 62.357) (end 224.282 62.357) (width 1.905) (layer B.Cu) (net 4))
 (segment (start 217.237919 97.79) (end 213.36 93.912081) (width 1.905) (layer B.Cu) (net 4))
 (segment (start 214.63 65.659) (end 217.932 62.357) (width 1.905) (layer B.Cu) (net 4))
 (segment (start 214.63 70.739) (end 214.63 65.659) (width 1.905) (layer B.Cu) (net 4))
 (segment (start 213.36 93.912081) (end 213.36 72.009) (width 1.905) (layer B.Cu) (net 4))
 (segment (start 218.44 97.79) (end 217.237919 97.79) (width 1.905) (layer B.Cu) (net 4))
 (segment (start 213.36 72.009) (end 214.63 70.739) (width 1.905) (layer B.Cu) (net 4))
 (segment (start 259.461 86.36) (end 256.2225 86.36) (width 1.905) (layer B.Cu) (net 4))
 (segment (start 256.2225 86.36) (end 252.73 86.36) (width 1.905) (layer B.Cu) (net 4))
 (segment (start 227.965 62.357) (end 229.235 63.627) (width 1.905) (layer B.Cu) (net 4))
 (segment (start 224.282 62.357) (end 227.965 62.357) (width 1.905) (layer B.Cu) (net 4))
 (segment (start 268.1605 77.6605) (end 259.461 86.36) (width 1.905) (layer B.Cu) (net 4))
 (segment (start 229.235 63.627) (end 244.094 63.627) (width 1.905) (layer B.Cu) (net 4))
 (segment (start 244.094 63.627) (end 248.285 59.436) (width 1.905) (layer B.Cu) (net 4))
 (segment (start 268.1605 64.3255) (end 268.1605 77.6605) (width 1.905) (layer B.Cu) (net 4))
 (segment (start 248.285 59.436) (end 263.271 59.436) (width 1.905) (layer B.Cu) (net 4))
 (segment (start 263.271 59.436) (end 268.1605 64.3255) (width 1.905) (layer B.Cu) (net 4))
 (segment (start 247.142 66.802) (end 244.348 69.596) (width 1.905) (layer B.Cu) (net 12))
 (segment (start 249.428 66.802) (end 247.142 66.802) (width 1.905) (layer B.Cu) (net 12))
 (segment (start 264.541 67.31) (end 264.541 65.532) (width 1.905) (layer B.Cu) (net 11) (status 10))
 (segment (start 264.541 65.532) (end 262.8265 63.8175) (width 1.905) (layer B.Cu) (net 11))
 (segment (start 258.9775 63.8175) (end 258.66 63.5) (width 1.905) (layer B.Cu) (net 11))
 (segment (start 262.8265 63.8175) (end 258.9775 63.8175) (width 1.905) (layer B.Cu) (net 11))
 (segment (start 258.66 63.5) (end 255.651 63.5) (width 1.905) (layer B.Cu) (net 11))
 (segment (start 254.254 64.897) (end 254.254 65.786) (width 1.905) (layer B.Cu) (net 11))
 (segment (start 255.651 63.5) (end 254.254 64.897) (width 1.905) (layer B.Cu) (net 11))
 (segment (start 255.485 78.74) (end 252.73 78.74) (width 1.905) (layer B.Cu) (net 3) (status 20))
 (segment (start 262.001 67.31) (end 262.001 72.224) (width 1.905) (layer B.Cu) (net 3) (status 10))
 (segment (start 262.001 72.224) (end 255.485 78.74) (width 1.905) (layer B.Cu) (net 3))
 (segment (start 237.557919 100.33) (end 237.430919 100.203) (width 1.905) (layer B.Cu) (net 9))
 (segment (start 238.76 100.33) (end 237.557919 100.33) (width 1.905) (layer B.Cu) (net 9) (status 10))
 (segment (start 237.430919 100.203) (end 236.982 100.203) (width 1.905) (layer B.Cu) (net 9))
 (segment (start 221.869 68.961) (end 232.791 79.883) (width 1.905) (layer B.Cu) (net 9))
 (segment (start 221.869 68.834) (end 221.869 68.961) (width 1.905) (layer B.Cu) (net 9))
 (segment (start 237.430919 100.203) (end 235.585 100.203) (width 1.905) (layer B.Cu) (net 9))
 (segment (start 232.791 97.409) (end 232.791 79.883) (width 1.905) (layer B.Cu) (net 9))
 (segment (start 235.585 100.203) (end 232.791 97.409) (width 1.905) (layer B.Cu) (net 9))
 (segment (start 244.475 54.2925) (end 244.348 54.4195) (width 1.905) (layer B.Cu) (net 13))
 (segment (start 254.762 54.2925) (end 244.475 54.2925) (width 1.905) (layer B.Cu) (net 13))
 (segment (start 258.247 54.2925) (end 260.025 52.5145) (width 1.905) (layer B.Cu) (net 13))
 (segment (start 254.762 54.2925) (end 258.247 54.2925) (width 1.905) (layer B.Cu) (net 13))
 (segment (start 216.789 59.182) (end 211.709 64.262) (width 1.905) (layer B.Cu) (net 13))
 (segment (start 211.709 64.262) (end 211.709 68.834) (width 1.905) (layer B.Cu) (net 13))
 (segment (start 228.854 59.182) (end 216.789 59.182) (width 1.905) (layer B.Cu) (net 13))
 (segment (start 244.348 57.7215) (end 244.348 54.4195) (width 1.905) (layer B.Cu) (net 13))
 (segment (start 242.404 59.6655) (end 244.348 57.7215) (width 1.905) (layer B.Cu) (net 13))
 (segment (start 229.3375 59.6655) (end 228.854 59.182) (width 1.905) (layer B.Cu) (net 13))
 (segment (start 242.404 59.6655) (end 229.3375 59.6655) (width 1.905) (layer B.Cu) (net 13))
 (segment (start 223.393 54.4195) (end 228.346 54.4195) (width 1.905) (layer B.Cu) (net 14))
 (segment (start 221.869 52.8955) (end 223.393 54.4195) (width 1.905) (layer B.Cu) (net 14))
 (segment (start 239.268 54.4195) (end 228.346 54.4195) (width 1.905) (layer B.Cu) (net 14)))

